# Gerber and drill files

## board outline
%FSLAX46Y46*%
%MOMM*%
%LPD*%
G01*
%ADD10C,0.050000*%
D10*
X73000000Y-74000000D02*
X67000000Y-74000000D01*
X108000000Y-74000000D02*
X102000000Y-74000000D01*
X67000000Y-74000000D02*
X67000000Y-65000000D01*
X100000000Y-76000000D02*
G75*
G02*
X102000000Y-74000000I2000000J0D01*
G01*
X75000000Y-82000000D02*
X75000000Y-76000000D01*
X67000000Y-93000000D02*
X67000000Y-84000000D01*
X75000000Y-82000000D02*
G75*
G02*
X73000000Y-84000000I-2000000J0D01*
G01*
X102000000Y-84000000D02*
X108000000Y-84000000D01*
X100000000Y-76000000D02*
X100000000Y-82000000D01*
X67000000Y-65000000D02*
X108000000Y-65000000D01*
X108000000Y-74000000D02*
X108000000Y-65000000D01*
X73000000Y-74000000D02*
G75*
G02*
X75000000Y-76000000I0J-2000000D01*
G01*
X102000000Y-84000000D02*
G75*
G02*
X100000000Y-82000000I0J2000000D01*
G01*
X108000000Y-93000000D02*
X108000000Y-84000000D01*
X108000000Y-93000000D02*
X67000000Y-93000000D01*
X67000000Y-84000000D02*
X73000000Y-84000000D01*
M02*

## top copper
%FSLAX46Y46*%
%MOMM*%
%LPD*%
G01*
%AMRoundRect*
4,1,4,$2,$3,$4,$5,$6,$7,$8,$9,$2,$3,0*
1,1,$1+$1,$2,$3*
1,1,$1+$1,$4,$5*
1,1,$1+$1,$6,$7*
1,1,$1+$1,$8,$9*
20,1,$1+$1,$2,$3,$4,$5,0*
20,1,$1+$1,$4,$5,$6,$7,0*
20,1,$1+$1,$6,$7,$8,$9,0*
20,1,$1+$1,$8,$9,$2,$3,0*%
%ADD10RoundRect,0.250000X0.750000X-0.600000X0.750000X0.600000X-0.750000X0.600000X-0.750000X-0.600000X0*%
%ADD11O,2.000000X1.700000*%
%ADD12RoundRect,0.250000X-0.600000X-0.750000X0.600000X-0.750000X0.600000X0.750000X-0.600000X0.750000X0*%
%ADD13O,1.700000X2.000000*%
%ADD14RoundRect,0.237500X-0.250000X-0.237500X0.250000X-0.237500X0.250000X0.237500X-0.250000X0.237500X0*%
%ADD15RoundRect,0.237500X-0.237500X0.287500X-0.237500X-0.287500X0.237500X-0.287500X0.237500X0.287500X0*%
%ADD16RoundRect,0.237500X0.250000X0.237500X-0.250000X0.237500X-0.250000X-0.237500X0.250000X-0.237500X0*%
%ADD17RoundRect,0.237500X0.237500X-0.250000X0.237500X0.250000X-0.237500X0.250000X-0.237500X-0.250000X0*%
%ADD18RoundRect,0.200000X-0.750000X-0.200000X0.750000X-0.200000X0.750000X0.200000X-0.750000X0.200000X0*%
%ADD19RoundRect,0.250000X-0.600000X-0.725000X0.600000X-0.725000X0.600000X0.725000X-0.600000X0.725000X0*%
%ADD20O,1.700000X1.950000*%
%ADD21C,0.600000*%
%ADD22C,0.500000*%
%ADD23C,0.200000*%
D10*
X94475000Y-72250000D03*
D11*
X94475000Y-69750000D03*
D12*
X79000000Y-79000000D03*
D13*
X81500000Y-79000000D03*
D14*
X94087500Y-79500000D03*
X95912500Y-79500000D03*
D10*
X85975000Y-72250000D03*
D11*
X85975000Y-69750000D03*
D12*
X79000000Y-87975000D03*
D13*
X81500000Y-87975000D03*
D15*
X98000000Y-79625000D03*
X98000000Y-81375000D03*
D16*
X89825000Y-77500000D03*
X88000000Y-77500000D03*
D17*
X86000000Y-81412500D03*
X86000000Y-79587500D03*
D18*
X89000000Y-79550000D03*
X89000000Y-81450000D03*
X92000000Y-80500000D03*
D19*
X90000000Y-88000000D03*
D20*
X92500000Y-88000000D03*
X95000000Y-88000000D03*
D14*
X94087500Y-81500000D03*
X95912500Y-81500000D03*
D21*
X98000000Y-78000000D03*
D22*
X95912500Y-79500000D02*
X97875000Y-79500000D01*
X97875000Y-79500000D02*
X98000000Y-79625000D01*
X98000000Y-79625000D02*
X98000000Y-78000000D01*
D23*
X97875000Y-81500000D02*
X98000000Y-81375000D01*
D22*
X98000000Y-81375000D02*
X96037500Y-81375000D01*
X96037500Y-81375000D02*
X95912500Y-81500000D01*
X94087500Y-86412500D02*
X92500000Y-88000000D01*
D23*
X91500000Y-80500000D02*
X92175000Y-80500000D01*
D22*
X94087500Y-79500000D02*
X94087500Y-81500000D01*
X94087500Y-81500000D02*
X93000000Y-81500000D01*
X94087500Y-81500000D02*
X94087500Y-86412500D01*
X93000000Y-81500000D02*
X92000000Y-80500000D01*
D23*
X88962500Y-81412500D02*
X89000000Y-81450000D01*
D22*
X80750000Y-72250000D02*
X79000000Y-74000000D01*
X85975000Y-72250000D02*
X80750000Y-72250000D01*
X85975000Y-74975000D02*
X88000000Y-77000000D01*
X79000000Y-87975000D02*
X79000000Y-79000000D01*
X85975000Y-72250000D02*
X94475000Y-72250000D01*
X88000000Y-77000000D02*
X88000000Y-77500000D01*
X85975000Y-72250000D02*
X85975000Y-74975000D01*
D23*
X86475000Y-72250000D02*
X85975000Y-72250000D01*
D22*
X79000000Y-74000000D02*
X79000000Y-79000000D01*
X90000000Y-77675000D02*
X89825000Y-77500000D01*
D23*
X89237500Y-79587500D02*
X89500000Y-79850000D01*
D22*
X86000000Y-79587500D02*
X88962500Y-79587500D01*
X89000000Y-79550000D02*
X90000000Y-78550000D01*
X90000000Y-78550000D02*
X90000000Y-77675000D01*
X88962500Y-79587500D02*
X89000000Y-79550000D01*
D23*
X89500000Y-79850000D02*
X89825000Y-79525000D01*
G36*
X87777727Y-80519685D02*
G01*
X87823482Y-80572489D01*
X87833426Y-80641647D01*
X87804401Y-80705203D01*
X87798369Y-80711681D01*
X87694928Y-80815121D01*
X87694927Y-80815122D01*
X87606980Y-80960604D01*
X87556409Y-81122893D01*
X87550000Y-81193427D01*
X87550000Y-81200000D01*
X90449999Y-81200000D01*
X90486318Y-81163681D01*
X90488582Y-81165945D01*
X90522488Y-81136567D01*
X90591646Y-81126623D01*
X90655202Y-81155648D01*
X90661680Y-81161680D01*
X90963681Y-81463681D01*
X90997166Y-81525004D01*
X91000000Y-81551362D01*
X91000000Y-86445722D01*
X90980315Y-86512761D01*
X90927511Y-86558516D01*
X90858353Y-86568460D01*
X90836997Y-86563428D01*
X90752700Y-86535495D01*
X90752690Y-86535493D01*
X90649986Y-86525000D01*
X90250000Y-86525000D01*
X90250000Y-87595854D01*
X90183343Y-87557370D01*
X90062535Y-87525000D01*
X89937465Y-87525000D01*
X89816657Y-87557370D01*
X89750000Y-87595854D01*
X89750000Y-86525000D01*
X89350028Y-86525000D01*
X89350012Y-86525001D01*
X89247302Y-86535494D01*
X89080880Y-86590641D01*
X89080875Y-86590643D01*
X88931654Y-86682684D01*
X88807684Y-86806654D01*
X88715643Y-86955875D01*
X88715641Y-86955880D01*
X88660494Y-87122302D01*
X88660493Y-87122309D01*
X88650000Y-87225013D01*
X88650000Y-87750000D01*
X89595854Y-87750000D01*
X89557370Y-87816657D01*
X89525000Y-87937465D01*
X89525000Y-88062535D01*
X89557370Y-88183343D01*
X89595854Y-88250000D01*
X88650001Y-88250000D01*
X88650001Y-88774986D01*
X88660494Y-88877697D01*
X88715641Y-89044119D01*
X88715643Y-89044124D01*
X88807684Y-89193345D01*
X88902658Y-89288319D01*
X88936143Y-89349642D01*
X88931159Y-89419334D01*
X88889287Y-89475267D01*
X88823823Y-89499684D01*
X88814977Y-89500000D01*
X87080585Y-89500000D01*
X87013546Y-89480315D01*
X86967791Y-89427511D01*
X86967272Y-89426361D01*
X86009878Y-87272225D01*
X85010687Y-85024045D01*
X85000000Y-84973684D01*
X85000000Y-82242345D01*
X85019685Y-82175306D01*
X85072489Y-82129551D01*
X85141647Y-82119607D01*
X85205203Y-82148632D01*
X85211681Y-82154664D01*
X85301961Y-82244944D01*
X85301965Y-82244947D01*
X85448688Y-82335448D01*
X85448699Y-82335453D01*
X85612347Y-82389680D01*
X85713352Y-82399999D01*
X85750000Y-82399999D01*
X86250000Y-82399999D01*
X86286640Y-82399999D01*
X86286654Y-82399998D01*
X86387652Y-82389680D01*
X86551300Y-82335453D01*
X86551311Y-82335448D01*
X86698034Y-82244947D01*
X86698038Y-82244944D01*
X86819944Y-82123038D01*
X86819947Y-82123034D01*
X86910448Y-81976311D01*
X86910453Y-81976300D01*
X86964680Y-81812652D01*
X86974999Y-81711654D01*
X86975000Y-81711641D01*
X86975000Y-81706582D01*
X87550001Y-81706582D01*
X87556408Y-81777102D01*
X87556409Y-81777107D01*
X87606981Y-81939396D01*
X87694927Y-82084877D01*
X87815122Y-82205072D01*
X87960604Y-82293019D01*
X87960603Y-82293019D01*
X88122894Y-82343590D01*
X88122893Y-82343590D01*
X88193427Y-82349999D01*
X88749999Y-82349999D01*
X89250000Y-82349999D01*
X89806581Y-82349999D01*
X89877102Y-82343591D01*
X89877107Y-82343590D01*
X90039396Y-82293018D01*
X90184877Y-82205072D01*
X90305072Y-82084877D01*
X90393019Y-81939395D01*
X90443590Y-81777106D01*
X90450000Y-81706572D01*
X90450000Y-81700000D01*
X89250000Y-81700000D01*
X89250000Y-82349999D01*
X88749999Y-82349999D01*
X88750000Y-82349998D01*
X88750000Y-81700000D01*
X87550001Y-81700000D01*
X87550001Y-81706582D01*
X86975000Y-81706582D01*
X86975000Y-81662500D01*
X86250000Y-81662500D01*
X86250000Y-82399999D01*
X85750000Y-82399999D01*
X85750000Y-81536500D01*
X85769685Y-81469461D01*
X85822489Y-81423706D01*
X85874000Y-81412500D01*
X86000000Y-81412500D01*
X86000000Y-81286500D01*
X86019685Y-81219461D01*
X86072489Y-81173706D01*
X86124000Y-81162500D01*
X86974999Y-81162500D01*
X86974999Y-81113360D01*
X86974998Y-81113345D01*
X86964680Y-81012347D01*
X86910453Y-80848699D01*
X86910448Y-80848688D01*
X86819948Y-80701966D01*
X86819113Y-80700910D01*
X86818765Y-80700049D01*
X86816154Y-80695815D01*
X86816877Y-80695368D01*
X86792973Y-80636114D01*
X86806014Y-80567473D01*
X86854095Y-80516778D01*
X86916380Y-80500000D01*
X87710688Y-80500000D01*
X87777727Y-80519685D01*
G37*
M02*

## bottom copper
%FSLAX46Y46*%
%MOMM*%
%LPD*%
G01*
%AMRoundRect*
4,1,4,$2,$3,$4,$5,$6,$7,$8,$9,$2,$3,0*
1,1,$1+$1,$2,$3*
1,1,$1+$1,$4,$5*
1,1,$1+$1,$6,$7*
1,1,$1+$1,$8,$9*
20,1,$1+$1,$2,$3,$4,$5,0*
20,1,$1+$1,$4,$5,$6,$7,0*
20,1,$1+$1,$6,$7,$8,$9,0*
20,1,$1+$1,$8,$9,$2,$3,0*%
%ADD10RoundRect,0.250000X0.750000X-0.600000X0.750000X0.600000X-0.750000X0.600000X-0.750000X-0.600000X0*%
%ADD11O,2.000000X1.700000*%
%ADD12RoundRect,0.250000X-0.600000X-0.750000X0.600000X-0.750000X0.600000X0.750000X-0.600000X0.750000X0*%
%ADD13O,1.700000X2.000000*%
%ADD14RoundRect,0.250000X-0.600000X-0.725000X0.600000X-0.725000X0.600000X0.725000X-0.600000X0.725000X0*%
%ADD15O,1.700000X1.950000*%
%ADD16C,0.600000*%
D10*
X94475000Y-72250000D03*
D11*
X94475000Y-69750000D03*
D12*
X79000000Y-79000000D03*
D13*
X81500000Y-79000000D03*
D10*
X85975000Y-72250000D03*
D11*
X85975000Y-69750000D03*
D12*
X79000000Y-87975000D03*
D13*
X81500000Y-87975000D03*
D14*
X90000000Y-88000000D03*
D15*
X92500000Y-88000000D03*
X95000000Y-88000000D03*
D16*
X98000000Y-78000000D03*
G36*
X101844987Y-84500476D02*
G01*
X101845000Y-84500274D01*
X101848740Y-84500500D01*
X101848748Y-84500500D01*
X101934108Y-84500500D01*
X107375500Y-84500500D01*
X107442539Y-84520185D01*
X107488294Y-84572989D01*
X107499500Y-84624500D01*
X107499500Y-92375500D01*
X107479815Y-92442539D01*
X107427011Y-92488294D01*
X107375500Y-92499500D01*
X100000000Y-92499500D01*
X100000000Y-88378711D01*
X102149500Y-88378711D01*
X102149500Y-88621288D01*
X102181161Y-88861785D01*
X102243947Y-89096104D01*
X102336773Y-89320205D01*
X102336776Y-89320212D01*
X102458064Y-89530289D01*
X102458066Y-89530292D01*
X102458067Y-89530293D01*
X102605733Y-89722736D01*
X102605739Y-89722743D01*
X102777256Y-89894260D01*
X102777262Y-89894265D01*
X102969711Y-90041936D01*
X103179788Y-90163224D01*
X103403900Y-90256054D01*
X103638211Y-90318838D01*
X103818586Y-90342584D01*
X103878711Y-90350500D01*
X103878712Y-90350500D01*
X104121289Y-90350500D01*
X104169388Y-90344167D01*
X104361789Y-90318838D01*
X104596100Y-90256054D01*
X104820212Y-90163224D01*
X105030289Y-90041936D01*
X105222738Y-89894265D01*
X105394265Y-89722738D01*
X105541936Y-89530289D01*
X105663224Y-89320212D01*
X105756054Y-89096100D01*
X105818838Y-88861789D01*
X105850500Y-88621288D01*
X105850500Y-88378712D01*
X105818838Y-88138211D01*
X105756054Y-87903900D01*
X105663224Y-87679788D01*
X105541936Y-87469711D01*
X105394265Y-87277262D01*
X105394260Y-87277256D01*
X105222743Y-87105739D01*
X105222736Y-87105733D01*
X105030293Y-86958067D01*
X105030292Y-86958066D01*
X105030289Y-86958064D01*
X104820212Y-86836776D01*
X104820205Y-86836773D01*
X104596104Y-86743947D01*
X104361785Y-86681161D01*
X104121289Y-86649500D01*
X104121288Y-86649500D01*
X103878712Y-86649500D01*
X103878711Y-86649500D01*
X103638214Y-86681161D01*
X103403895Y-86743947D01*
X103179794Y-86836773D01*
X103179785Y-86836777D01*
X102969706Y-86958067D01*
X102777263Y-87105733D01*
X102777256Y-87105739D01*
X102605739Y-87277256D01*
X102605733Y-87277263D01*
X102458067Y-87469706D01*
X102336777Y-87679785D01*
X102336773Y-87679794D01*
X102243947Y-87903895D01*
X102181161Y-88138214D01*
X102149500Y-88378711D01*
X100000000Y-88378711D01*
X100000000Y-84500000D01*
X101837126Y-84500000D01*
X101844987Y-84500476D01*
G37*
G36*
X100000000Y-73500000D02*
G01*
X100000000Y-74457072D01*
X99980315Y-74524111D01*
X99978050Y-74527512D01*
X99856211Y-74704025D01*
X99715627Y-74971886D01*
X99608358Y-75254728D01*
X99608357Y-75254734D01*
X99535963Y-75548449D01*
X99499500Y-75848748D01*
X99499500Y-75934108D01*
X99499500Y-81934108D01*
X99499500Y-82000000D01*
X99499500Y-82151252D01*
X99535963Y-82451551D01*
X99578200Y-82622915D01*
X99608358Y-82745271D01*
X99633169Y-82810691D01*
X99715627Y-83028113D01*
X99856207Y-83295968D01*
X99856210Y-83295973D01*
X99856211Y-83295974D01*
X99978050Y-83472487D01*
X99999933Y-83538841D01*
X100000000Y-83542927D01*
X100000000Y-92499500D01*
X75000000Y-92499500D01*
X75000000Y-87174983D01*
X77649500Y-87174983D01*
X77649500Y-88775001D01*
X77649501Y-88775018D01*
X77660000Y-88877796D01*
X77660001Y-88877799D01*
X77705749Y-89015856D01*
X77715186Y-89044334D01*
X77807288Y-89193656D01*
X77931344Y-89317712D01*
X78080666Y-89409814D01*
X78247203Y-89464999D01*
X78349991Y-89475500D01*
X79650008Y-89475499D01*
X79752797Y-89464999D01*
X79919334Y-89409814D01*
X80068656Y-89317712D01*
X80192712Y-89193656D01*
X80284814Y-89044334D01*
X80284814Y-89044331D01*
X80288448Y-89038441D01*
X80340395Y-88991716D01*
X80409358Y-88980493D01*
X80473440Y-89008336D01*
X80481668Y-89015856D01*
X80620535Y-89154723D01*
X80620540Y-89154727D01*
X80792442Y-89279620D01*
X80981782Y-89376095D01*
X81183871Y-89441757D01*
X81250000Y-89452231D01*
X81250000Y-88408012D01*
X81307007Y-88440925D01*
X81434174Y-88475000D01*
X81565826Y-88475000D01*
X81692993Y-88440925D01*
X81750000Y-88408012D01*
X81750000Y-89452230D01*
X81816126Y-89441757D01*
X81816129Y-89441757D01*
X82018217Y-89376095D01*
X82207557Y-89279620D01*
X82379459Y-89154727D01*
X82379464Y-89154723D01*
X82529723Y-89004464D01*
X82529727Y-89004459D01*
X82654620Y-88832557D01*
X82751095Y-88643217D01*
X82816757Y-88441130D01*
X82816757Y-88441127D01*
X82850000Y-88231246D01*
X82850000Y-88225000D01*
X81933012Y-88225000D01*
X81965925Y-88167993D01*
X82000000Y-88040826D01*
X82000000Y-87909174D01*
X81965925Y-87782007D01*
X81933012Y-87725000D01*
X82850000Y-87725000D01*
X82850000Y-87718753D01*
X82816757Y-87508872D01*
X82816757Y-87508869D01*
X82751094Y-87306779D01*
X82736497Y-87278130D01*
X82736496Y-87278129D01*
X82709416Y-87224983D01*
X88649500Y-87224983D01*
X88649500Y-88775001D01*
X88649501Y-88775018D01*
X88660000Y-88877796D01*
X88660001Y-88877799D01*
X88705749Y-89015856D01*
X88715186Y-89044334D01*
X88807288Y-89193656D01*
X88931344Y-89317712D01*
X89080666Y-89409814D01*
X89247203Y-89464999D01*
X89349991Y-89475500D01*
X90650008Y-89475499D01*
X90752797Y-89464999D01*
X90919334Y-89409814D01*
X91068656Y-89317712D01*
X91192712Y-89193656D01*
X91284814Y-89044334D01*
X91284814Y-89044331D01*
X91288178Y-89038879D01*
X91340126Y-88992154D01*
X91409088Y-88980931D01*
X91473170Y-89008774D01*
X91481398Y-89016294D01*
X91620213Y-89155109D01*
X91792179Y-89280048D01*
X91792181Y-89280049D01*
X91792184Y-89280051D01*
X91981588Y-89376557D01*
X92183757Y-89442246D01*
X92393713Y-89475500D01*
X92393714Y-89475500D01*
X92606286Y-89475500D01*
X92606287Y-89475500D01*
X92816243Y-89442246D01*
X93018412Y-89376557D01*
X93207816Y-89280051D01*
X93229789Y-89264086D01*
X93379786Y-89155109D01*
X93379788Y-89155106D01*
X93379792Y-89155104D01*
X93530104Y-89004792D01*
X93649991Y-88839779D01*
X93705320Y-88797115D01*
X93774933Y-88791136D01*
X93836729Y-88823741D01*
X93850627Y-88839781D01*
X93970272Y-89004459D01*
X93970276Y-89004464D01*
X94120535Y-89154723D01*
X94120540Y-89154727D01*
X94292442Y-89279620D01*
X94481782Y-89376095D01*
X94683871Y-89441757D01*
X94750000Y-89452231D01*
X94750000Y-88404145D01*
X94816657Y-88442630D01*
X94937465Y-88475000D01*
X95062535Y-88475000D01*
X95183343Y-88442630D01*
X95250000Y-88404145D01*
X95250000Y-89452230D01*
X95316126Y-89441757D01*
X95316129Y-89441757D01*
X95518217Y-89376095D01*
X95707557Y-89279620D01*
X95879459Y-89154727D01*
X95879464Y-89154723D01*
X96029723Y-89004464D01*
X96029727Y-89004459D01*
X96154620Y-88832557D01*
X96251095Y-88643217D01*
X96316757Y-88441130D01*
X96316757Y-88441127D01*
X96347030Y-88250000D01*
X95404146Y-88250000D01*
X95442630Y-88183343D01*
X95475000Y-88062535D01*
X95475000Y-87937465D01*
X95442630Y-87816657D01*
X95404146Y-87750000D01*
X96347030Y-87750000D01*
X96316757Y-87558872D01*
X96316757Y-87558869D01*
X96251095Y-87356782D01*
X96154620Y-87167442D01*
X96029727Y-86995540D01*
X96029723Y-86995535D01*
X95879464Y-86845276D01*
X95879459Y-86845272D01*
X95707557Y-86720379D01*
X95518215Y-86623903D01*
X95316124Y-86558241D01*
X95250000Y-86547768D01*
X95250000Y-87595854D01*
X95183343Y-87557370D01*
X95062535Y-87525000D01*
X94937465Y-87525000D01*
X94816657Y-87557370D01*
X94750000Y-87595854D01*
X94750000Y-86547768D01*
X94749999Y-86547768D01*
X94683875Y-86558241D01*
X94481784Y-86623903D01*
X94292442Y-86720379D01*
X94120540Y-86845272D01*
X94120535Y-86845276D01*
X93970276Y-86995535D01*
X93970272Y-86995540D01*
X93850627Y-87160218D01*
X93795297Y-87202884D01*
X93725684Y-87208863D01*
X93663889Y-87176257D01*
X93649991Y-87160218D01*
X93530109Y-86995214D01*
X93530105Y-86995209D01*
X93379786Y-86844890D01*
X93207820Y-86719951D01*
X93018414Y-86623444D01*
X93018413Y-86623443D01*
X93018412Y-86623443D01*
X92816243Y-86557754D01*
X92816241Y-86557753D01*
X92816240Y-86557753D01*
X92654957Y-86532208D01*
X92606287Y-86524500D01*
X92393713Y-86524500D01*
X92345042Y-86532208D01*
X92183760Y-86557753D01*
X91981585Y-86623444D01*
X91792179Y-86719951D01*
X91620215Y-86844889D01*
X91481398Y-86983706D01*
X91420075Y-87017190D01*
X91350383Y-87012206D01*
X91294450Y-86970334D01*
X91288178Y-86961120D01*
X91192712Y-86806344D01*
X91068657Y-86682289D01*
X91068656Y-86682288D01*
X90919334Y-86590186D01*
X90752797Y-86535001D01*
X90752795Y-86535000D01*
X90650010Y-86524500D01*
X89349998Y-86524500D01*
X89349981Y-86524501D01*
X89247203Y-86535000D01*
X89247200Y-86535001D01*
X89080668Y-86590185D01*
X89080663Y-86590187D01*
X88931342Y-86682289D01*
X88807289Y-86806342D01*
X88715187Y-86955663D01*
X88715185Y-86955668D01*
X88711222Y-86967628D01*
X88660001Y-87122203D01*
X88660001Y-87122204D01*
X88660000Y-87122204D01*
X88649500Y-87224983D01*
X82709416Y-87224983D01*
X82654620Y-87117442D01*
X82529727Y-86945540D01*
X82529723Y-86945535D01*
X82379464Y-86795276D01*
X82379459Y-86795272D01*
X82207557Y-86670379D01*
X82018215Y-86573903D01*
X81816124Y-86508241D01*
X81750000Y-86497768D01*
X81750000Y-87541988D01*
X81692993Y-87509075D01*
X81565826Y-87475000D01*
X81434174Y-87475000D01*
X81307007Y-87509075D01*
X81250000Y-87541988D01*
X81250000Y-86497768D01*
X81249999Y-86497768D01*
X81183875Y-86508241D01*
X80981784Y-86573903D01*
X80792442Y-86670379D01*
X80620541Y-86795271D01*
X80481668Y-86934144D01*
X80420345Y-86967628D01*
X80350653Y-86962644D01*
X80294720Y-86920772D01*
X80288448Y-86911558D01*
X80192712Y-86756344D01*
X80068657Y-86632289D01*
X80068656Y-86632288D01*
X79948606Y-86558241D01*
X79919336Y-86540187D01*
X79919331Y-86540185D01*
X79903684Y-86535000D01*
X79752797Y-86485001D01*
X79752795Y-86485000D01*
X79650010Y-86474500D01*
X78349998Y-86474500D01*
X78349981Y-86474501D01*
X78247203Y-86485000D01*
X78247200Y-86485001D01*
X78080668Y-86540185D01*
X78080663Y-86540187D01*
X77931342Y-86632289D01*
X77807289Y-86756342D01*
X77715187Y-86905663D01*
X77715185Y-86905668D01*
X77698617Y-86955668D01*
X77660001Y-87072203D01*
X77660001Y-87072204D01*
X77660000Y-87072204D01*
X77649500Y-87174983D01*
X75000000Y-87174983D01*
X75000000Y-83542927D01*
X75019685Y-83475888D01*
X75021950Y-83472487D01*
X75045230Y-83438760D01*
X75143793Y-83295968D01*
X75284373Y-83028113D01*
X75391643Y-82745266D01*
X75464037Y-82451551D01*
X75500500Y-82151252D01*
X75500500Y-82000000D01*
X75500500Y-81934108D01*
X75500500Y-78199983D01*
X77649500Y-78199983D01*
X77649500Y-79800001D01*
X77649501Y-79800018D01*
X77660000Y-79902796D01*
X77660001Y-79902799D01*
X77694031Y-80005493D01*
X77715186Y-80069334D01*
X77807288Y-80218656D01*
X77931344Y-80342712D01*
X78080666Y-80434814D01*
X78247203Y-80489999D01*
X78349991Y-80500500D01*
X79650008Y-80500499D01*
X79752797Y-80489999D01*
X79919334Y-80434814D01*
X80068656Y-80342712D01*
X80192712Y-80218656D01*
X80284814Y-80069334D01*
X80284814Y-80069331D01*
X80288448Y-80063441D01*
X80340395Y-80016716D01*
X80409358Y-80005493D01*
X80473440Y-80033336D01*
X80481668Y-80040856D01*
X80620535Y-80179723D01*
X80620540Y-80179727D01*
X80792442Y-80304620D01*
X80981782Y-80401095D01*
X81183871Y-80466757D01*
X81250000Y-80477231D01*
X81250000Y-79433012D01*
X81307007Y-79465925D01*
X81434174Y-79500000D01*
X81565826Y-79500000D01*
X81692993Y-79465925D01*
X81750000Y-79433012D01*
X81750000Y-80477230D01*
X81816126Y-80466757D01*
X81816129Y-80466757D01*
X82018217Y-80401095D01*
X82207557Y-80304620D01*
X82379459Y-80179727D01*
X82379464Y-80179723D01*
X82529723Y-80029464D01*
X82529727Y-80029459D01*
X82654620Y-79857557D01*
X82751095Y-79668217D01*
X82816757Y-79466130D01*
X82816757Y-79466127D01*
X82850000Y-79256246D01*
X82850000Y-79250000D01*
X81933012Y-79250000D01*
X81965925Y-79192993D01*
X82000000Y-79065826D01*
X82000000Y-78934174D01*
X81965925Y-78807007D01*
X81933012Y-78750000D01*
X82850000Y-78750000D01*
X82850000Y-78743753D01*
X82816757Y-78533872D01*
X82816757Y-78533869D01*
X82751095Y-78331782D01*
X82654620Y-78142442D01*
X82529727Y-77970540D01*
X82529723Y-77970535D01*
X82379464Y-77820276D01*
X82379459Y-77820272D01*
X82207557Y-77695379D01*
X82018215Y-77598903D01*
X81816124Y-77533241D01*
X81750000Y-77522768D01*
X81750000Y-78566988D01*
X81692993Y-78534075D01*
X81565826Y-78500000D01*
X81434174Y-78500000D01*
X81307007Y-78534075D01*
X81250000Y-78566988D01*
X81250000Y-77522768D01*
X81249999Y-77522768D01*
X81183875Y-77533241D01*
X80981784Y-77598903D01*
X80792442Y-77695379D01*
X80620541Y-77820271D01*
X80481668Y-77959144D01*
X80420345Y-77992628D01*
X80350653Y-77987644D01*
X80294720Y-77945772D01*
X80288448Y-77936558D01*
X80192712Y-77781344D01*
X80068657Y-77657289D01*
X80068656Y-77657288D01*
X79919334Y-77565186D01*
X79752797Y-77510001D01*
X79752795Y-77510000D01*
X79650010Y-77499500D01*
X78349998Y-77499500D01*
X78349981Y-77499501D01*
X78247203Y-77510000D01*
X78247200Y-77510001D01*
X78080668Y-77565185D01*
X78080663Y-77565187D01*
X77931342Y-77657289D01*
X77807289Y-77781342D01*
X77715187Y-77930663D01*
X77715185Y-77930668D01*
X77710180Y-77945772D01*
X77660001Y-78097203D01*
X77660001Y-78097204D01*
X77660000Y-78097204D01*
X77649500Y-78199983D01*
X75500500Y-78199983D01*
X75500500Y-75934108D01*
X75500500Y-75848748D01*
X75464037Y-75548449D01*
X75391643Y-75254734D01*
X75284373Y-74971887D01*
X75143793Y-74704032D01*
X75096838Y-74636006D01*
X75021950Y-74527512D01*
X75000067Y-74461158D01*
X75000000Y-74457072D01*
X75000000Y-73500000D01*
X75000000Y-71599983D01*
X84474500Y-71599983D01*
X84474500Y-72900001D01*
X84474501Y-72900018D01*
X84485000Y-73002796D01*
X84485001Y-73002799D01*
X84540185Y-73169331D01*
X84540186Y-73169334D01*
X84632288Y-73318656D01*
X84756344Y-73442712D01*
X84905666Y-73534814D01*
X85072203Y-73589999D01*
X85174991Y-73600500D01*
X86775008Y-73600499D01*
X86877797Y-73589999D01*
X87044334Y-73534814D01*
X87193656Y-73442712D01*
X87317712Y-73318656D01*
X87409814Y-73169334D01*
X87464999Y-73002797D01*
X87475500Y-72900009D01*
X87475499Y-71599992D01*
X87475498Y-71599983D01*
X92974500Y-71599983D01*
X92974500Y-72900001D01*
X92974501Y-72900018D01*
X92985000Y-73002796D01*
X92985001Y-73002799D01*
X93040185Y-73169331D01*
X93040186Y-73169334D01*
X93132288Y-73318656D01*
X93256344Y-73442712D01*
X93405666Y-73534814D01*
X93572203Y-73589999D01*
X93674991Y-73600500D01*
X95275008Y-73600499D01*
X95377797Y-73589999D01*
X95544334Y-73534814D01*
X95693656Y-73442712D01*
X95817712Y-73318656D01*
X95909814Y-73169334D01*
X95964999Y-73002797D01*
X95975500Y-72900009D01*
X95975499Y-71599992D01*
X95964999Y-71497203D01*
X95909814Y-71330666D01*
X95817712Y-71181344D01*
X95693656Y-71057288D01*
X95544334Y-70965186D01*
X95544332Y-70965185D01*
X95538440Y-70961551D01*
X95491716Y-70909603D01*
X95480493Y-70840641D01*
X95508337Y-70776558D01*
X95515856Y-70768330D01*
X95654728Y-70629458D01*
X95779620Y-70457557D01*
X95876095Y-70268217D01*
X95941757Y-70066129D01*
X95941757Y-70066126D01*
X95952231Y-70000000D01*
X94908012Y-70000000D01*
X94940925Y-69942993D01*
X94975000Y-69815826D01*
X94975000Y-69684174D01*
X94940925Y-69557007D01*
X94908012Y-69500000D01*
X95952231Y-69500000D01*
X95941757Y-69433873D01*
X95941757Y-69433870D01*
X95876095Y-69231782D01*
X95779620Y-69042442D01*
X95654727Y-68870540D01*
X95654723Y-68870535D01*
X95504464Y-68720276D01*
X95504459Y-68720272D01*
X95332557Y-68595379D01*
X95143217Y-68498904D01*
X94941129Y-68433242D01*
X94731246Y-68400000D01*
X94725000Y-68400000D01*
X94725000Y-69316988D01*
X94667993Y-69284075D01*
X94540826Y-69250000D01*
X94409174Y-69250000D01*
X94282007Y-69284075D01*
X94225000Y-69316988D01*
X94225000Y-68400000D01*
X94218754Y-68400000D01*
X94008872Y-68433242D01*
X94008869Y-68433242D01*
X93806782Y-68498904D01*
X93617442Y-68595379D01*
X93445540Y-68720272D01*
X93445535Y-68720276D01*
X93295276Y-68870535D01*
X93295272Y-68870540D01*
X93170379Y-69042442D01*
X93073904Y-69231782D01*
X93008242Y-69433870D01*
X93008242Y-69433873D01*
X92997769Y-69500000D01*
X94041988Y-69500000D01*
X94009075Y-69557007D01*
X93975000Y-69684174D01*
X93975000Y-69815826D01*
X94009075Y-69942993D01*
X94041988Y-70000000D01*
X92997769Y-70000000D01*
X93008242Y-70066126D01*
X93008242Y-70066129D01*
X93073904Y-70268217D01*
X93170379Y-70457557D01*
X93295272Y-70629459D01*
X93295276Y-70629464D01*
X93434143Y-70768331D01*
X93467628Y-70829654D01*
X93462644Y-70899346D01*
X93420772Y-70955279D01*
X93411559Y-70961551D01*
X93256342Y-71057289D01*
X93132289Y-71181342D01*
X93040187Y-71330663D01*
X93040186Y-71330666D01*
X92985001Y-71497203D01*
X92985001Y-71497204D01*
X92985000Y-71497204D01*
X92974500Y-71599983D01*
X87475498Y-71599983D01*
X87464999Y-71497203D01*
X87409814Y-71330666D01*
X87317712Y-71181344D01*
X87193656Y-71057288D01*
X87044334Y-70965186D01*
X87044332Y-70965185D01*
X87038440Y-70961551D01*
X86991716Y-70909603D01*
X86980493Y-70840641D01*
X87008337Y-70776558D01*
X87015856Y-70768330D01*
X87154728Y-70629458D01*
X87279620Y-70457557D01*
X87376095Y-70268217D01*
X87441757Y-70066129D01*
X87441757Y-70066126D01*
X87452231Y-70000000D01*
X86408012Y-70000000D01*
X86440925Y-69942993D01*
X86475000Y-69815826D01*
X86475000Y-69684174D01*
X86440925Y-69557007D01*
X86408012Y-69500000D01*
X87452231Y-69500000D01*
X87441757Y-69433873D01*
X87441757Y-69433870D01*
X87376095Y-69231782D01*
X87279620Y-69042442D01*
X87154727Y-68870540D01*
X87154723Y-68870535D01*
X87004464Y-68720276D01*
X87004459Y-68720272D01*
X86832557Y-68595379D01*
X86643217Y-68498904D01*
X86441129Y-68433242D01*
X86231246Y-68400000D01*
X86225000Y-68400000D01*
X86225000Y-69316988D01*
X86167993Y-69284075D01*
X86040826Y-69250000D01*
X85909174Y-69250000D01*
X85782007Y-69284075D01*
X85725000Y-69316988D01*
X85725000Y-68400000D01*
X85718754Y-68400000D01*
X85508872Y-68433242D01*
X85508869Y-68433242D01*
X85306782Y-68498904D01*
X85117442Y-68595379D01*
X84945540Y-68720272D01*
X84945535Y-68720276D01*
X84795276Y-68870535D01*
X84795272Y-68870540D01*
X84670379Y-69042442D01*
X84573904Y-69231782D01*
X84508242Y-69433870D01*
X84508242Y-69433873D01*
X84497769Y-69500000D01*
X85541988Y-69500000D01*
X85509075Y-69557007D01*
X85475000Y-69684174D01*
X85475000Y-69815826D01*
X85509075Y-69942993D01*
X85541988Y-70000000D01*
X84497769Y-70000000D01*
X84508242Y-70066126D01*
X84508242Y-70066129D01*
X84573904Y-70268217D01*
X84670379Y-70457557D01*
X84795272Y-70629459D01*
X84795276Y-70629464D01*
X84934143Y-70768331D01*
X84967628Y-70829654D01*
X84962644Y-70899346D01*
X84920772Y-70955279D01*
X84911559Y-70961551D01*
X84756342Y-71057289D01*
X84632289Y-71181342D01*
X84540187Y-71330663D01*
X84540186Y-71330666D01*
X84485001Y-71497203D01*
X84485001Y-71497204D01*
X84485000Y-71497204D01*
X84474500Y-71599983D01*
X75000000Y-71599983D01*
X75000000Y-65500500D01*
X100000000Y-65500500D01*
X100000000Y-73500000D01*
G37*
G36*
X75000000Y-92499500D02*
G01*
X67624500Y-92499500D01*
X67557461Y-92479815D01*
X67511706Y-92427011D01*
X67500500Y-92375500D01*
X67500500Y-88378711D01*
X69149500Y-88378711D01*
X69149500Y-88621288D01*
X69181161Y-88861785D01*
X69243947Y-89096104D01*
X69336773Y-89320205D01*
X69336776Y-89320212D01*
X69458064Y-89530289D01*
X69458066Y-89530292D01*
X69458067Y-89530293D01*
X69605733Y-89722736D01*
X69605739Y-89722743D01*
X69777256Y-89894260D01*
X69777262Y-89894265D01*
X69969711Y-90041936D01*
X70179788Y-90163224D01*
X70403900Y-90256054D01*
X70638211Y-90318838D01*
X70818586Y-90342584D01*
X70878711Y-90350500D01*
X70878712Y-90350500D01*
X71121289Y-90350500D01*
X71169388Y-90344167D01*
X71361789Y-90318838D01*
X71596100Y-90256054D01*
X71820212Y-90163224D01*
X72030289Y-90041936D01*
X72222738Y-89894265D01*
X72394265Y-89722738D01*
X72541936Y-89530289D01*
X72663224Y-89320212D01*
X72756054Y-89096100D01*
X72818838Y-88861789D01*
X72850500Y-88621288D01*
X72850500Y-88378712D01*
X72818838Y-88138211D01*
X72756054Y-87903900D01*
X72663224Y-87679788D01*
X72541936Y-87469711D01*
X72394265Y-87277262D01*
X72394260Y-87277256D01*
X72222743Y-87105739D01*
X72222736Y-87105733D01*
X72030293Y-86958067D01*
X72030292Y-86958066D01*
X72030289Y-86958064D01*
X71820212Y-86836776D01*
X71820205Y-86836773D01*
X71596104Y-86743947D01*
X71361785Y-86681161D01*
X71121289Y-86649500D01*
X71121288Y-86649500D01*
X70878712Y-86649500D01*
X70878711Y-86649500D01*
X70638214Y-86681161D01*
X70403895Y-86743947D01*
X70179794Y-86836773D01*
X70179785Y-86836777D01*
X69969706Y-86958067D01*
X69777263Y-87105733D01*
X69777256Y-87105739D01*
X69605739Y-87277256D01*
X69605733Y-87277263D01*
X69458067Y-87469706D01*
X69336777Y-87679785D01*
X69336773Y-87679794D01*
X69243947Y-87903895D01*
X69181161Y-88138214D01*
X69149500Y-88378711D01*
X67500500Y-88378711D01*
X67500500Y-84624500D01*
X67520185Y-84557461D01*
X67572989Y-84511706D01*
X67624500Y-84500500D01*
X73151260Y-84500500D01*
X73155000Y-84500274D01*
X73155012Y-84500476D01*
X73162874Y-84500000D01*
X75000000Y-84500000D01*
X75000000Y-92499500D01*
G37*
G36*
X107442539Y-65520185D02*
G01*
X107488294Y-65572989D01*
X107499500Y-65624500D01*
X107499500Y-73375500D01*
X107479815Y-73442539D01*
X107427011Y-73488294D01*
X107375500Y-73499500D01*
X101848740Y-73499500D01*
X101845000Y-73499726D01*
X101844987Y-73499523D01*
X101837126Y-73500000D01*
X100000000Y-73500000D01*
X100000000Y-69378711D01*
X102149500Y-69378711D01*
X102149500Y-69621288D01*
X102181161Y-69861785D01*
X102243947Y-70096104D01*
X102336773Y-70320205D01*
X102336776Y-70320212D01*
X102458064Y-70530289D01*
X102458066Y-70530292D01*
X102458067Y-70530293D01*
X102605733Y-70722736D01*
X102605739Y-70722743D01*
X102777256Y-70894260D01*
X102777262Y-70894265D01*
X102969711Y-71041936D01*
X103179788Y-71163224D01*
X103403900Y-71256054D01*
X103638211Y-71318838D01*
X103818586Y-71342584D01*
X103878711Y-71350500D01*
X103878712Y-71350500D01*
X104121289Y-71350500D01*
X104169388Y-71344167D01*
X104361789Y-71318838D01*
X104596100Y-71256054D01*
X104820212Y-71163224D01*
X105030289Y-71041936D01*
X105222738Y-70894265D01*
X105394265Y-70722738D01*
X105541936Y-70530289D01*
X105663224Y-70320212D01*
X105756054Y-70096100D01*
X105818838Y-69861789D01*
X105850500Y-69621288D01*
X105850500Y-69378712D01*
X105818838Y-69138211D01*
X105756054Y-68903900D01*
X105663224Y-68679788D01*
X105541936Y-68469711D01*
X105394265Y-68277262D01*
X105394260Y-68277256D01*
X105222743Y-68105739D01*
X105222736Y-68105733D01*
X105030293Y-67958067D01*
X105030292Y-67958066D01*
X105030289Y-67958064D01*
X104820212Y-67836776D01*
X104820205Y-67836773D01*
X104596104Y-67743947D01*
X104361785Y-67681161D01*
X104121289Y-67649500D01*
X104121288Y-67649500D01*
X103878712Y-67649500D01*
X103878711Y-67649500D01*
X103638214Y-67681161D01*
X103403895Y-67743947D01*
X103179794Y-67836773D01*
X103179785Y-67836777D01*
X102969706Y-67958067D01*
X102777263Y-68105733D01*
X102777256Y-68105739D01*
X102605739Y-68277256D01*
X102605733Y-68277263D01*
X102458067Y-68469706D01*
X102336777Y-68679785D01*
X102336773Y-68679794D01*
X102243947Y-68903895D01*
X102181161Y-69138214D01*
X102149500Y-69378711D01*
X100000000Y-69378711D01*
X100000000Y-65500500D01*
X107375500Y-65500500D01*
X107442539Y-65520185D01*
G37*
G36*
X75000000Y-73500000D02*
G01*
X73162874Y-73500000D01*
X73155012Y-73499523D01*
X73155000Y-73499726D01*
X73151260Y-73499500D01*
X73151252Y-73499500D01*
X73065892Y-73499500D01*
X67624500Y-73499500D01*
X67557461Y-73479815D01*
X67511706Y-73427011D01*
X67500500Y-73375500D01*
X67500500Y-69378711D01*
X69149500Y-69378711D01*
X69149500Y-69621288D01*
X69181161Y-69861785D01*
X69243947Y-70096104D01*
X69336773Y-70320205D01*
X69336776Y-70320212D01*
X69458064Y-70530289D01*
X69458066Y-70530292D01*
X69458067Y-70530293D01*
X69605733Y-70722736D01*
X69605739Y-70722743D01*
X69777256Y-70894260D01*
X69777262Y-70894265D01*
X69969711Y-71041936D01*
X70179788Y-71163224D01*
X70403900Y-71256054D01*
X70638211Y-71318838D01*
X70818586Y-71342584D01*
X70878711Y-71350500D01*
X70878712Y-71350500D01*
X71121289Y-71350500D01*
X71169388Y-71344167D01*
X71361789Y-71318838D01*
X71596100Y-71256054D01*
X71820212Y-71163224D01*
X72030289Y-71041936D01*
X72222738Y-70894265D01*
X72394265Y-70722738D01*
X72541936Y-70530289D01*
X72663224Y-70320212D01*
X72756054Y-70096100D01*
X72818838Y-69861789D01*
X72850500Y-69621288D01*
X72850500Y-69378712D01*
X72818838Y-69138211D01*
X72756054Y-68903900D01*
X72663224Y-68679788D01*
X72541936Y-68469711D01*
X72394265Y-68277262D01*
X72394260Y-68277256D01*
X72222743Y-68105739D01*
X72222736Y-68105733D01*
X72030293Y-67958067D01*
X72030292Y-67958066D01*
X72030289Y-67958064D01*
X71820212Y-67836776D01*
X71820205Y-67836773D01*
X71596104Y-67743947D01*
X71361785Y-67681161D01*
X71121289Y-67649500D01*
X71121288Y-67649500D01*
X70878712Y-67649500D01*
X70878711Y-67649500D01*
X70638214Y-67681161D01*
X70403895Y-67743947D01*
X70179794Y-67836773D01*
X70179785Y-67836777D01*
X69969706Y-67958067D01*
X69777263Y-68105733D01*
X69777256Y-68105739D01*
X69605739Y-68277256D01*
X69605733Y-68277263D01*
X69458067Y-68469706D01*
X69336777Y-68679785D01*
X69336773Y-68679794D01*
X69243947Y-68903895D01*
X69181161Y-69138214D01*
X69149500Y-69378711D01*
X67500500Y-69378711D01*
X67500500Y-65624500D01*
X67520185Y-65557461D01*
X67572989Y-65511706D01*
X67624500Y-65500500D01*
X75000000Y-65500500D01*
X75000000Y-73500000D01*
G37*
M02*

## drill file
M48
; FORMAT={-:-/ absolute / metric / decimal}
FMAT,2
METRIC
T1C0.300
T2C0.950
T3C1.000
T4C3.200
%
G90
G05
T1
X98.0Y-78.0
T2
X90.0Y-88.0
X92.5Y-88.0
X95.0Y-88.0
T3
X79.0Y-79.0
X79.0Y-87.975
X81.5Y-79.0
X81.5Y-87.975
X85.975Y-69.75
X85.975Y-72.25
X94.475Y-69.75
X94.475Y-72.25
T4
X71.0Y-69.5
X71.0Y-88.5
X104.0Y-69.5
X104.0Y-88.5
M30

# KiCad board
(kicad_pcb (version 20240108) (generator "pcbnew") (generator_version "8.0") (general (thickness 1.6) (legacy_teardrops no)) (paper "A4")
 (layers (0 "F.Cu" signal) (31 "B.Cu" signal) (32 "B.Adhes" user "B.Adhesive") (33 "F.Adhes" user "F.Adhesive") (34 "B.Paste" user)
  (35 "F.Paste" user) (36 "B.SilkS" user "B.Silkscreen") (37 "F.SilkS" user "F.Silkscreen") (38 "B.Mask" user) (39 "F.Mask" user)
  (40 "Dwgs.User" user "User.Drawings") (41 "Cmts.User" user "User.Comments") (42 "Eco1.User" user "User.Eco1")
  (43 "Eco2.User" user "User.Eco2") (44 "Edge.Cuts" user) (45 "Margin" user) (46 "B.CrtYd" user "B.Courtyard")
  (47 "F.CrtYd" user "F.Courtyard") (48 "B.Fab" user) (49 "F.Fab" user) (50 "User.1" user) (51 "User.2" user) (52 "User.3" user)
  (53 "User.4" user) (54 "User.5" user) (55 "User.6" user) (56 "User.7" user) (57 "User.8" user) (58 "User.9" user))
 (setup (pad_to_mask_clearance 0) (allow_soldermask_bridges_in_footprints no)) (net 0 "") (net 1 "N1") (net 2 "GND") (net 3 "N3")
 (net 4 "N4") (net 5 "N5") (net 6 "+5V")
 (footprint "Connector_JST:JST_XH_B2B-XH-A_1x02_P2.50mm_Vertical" (layer "F.Cu") (at 94.475 72.25 90)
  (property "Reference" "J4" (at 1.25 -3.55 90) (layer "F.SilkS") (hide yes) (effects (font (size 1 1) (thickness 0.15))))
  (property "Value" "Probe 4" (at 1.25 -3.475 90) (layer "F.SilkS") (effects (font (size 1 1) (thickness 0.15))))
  (pad "1" thru_hole roundrect (at 0 0 90) (size 1.7 2) (drill 1) (layers "*.Cu" "*.Mask") (remove_unused_layers no)
   (roundrect_rratio 0.147059) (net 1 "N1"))
  (pad "2" thru_hole oval (at 2.5 0 90) (size 1.7 2) (drill 1) (layers "*.Cu" "*.Mask") (remove_unused_layers no) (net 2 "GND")))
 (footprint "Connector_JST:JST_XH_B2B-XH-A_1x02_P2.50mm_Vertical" (layer "F.Cu") (at 79 79)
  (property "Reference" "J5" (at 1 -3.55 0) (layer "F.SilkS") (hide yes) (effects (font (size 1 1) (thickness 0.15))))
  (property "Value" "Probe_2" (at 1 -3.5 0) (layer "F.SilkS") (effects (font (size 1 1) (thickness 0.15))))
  (pad "1" thru_hole roundrect (at 0 0) (size 1.7 2) (drill 1) (layers "*.Cu" "*.Mask") (remove_unused_layers no)
   (roundrect_rratio 0.147059) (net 1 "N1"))
  (pad "2" thru_hole oval (at 2.5 0) (size 1.7 2) (drill 1) (layers "*.Cu" "*.Mask") (remove_unused_layers no) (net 2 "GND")))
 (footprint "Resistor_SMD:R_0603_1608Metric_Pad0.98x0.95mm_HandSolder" (layer "F.Cu") (at 95 79.5)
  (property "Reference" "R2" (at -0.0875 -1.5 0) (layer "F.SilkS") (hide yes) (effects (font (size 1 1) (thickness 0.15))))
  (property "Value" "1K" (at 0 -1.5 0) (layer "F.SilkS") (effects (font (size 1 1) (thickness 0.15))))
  (pad "1" smd roundrect (at -0.9125 0) (size 0.975 0.95) (layers "F.Cu" "F.Paste" "F.Mask") (roundrect_rratio 0.25) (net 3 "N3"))
  (pad "2" smd roundrect (at 0.9125 0) (size 0.975 0.95) (layers "F.Cu" "F.Paste" "F.Mask") (roundrect_rratio 0.25) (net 2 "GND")))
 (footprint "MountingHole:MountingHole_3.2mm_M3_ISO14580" (layer "F.Cu") (at 71 88.5)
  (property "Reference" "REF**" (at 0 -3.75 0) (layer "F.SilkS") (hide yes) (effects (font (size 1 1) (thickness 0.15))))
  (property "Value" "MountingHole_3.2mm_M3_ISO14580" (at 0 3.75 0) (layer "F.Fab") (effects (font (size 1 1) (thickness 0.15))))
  (pad "" np_thru_hole circle (at 0 0) (size 3.2 3.2) (drill 3.2) (layers "*.Cu" "*.Mask")))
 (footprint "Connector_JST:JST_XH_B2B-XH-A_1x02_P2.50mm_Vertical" (layer "F.Cu") (at 85.975 72.25 90)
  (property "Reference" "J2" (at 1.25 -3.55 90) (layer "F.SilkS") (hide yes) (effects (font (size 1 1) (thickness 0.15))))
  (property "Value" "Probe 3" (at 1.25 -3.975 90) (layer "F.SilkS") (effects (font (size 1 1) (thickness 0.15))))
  (pad "1" thru_hole roundrect (at 0 0 90) (size 1.7 2) (drill 1) (layers "*.Cu" "*.Mask") (remove_unused_layers no)
   (roundrect_rratio 0.147059) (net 1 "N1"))
  (pad "2" thru_hole oval (at 2.5 0 90) (size 1.7 2) (drill 1) (layers "*.Cu" "*.Mask") (remove_unused_layers no) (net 2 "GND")))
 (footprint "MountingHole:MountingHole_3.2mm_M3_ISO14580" (layer "F.Cu") (at 71 69.5)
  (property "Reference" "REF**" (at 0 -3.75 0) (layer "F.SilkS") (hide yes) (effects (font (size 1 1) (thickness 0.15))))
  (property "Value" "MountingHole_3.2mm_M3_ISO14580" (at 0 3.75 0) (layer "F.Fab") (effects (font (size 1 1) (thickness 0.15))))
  (pad "" np_thru_hole circle (at 0 0) (size 3.2 3.2) (drill 3.2) (layers "*.Cu" "*.Mask")))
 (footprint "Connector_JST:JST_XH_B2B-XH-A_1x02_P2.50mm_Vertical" (layer "F.Cu") (at 79 87.975)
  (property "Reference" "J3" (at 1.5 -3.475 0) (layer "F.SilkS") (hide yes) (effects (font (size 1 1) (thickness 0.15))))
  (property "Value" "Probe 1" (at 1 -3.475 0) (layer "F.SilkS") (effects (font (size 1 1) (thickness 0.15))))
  (pad "1" thru_hole roundrect (at 0 0) (size 1.7 2) (drill 1) (layers "*.Cu" "*.Mask") (remove_unused_layers no)
   (roundrect_rratio 0.147059) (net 1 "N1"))
  (pad "2" thru_hole oval (at 2.5 0) (size 1.7 2) (drill 1) (layers "*.Cu" "*.Mask") (remove_unused_layers no) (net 2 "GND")))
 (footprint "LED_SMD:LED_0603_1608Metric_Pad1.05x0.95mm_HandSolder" (layer "F.Cu") (at 98 80.5 -90)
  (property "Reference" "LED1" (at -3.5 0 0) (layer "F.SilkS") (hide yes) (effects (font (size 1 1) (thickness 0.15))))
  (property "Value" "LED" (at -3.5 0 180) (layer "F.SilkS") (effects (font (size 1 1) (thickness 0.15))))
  (pad "1" smd roundrect (at -0.875 0 270) (size 1.05 0.95) (layers "F.Cu" "F.Paste" "F.Mask") (roundrect_rratio 0.25) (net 2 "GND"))
  (pad "2" smd roundrect (at 0.875 0 270) (size 1.05 0.95) (layers "F.Cu" "F.Paste" "F.Mask") (roundrect_rratio 0.25) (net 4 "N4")))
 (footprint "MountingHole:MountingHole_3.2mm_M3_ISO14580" (layer "F.Cu") (at 104 88.5)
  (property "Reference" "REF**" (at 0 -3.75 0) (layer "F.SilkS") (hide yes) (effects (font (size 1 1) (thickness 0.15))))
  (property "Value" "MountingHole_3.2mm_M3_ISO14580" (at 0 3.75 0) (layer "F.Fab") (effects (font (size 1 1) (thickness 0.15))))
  (pad "" np_thru_hole circle (at 0 0) (size 3.2 3.2) (drill 3.2) (layers "*.Cu" "*.Mask")))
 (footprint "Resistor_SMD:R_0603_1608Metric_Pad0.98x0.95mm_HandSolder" (layer "F.Cu") (at 88.9125 77.5 180)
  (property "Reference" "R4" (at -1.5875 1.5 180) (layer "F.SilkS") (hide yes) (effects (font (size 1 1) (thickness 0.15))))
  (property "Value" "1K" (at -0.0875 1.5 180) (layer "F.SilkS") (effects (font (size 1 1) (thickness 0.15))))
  (pad "1" smd roundrect (at -0.9125 0 180) (size 0.975 0.95) (layers "F.Cu" "F.Paste" "F.Mask") (roundrect_rratio 0.25) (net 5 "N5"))
  (pad "2" smd roundrect (at 0.9125 0 180) (size 0.975 0.95) (layers "F.Cu" "F.Paste" "F.Mask") (roundrect_rratio 0.25) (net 1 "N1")))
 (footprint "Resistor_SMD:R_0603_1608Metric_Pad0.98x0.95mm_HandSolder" (layer "F.Cu") (at 86 80.5 90)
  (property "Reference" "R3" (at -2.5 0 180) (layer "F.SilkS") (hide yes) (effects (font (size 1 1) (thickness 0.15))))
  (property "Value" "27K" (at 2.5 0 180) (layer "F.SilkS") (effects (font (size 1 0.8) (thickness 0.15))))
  (pad "1" smd roundrect (at -0.9125 0 90) (size 0.975 0.95) (layers "F.Cu" "F.Paste" "F.Mask") (roundrect_rratio 0.25) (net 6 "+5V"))
  (pad "2" smd roundrect (at 0.9125 0 90) (size 0.975 0.95) (layers "F.Cu" "F.Paste" "F.Mask") (roundrect_rratio 0.25) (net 5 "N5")))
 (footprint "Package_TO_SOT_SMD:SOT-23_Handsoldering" (layer "F.Cu") (at 90.5 80.5)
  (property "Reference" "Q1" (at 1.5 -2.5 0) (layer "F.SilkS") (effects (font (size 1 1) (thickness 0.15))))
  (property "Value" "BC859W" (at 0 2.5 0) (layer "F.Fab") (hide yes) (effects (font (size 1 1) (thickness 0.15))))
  (pad "1" smd roundrect (at -1.5 -0.95) (size 1.9 0.8) (layers "F.Cu" "F.Paste" "F.Mask") (roundrect_rratio 0.25) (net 5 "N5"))
  (pad "2" smd roundrect (at -1.5 0.95) (size 1.9 0.8) (layers "F.Cu" "F.Paste" "F.Mask") (roundrect_rratio 0.25) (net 6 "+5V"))
  (pad "3" smd roundrect (at 1.5 0) (size 1.9 0.8) (layers "F.Cu" "F.Paste" "F.Mask") (roundrect_rratio 0.25) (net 3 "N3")))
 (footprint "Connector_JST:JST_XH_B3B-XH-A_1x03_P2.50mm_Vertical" (layer "F.Cu") (at 90 88)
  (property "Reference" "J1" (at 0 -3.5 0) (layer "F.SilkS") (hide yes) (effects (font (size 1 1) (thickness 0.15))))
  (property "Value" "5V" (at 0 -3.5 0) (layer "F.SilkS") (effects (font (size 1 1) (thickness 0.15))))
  (pad "1" thru_hole roundrect (at 0 0) (size 1.7 1.95) (drill 0.95) (layers "*.Cu" "*.Mask") (remove_unused_layers no)
   (roundrect_rratio 0.147059) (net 6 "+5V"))
  (pad "2" thru_hole oval (at 2.5 0) (size 1.7 1.95) (drill 0.95) (layers "*.Cu" "*.Mask") (remove_unused_layers no) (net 3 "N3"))
  (pad "3" thru_hole oval (at 5 0) (size 1.7 1.95) (drill 0.95) (layers "*.Cu" "*.Mask") (remove_unused_layers no) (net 2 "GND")))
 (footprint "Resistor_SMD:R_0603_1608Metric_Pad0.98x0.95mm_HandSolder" (layer "F.Cu") (at 95 81.5)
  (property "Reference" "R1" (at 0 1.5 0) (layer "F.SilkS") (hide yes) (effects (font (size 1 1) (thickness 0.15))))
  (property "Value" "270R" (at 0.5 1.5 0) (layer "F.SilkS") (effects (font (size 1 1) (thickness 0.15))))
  (pad "1" smd roundrect (at -0.9125 0) (size 0.975 0.95) (layers "F.Cu" "F.Paste" "F.Mask") (roundrect_rratio 0.25) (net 3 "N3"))
  (pad "2" smd roundrect (at 0.9125 0) (size 0.975 0.95) (layers "F.Cu" "F.Paste" "F.Mask") (roundrect_rratio 0.25) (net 4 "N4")))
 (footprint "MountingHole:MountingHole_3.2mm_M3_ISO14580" (layer "F.Cu") (at 104 69.5)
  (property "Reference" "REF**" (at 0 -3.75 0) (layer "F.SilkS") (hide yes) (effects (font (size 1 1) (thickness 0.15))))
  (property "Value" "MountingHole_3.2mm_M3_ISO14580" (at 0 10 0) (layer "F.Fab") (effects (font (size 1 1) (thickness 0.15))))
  (pad "" np_thru_hole circle (at 0 0) (size 3.2 3.2) (drill 3.2) (layers "*.Cu" "*.Mask")))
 (gr_line (start 73 74) (end 67 74) (stroke (width 0.05) (type default)) (layer "Edge.Cuts"))
 (gr_line (start 108 74) (end 102 74) (stroke (width 0.05) (type default)) (layer "Edge.Cuts"))
 (gr_line (start 67 74) (end 67 65) (stroke (width 0.05) (type default)) (layer "Edge.Cuts"))
 (gr_arc (start 100 76) (mid 100.585786 74.585786) (end 102 74) (stroke (width 0.05) (type default)) (layer "Edge.Cuts"))
 (gr_line (start 75 82) (end 75 76) (stroke (width 0.05) (type default)) (layer "Edge.Cuts"))
 (gr_line (start 67 93) (end 67 84) (stroke (width 0.05) (type default)) (layer "Edge.Cuts"))
 (gr_arc (start 75 82) (mid 74.414214 83.414214) (end 73 84) (stroke (width 0.05) (type default)) (layer "Edge.Cuts"))
 (gr_line (start 102 84) (end 108 84) (stroke (width 0.05) (type default)) (layer "Edge.Cuts"))
 (gr_line (start 100 76) (end 100 82) (stroke (width 0.05) (type default)) (layer "Edge.Cuts"))
 (gr_line (start 67 65) (end 108 65) (stroke (width 0.05) (type default)) (layer "Edge.Cuts"))
 (gr_line (start 108 74) (end 108 65) (stroke (width 0.05) (type default)) (layer "Edge.Cuts"))
 (gr_arc (start 73 74) (mid 74.414214 74.585786) (end 75 76) (stroke (width 0.05) (type default)) (layer "Edge.Cuts"))
 (gr_arc (start 102 84) (mid 100.585786 83.414214) (end 100 82) (stroke (width 0.05) (type default)) (layer "Edge.Cuts"))
 (gr_line (start 108 93) (end 108 84) (stroke (width 0.05) (type default)) (layer "Edge.Cuts"))
 (gr_line (start 108 93) (end 67 93) (stroke (width 0.05) (type default)) (layer "Edge.Cuts"))
 (gr_line (start 67 84) (end 73 84) (stroke (width 0.05) (type default)) (layer "Edge.Cuts"))
 (segment (start 95.9125 79.5) (end 97.875 79.5) (width 0.5) (layer "F.Cu") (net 2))
 (segment (start 97.875 79.5) (end 98 79.625) (width 0.5) (layer "F.Cu") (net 2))
 (segment (start 98 79.625) (end 98 78) (width 0.5) (layer "F.Cu") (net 2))
 (via (at 98 78) (size 0.6) (drill 0.3) (layers "F.Cu" "B.Cu") (free yes) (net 2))
 (segment (start 97.875 81.5) (end 98 81.375) (width 0.2) (layer "F.Cu") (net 4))
 (segment (start 98 81.375) (end 96.0375 81.375) (width 0.5) (layer "F.Cu") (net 4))
 (segment (start 96.0375 81.375) (end 95.9125 81.5) (width 0.5) (layer "F.Cu") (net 4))
 (segment (start 94.0875 86.4125) (end 92.5 88) (width 0.5) (layer "F.Cu") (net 3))
 (segment (start 91.5 80.5) (end 92.175 80.5) (width 0.2) (layer "F.Cu") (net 3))
 (segment (start 94.0875 79.5) (end 94.0875 81.5) (width 0.5) (layer "F.Cu") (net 3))
 (segment (start 94.0875 81.5) (end 93 81.5) (width 0.5) (layer "F.Cu") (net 3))
 (segment (start 94.0875 81.5) (end 94.0875 86.4125) (width 0.5) (layer "F.Cu") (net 3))
 (segment (start 93 81.5) (end 92 80.5) (width 0.5) (layer "F.Cu") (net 3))
 (segment (start 88.9625 81.4125) (end 89 81.45) (width 0.2) (layer "F.Cu") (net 6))
 (segment (start 80.75 72.25) (end 79 74) (width 0.5) (layer "F.Cu") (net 1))
 (segment (start 85.975 72.25) (end 80.75 72.25) (width 0.5) (layer "F.Cu") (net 1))
 (segment (start 85.975 74.975) (end 88 77) (width 0.5) (layer "F.Cu") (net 1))
 (segment (start 79 87.975) (end 79 79) (width 0.5) (layer "F.Cu") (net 1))
 (segment (start 85.975 72.25) (end 94.475 72.25) (width 0.5) (layer "F.Cu") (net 1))
 (segment (start 88 77) (end 88 77.5) (width 0.5) (layer "F.Cu") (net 1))
 (segment (start 85.975 72.25) (end 85.975 74.975) (width 0.5) (layer "F.Cu") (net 1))
 (segment (start 86.475 72.25) (end 85.975 72.25) (width 0.2) (layer "F.Cu") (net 1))
 (segment (start 79 74) (end 79 79) (width 0.5) (layer "F.Cu") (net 1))
 (segment (start 90 77.675) (end 89.825 77.5) (width 0.5) (layer "F.Cu") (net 5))
 (segment (start 89.2375 79.5875) (end 89.5 79.85) (width 0.2) (layer "F.Cu") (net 5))
 (segment (start 86 79.5875) (end 88.9625 79.5875) (width 0.5) (layer "F.Cu") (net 5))
 (segment (start 89 79.55) (end 90 78.55) (width 0.5) (layer "F.Cu") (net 5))
 (segment (start 90 78.55) (end 90 77.675) (width 0.5) (layer "F.Cu") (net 5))
 (segment (start 88.9625 79.5875) (end 89 79.55) (width 0.5) (layer "F.Cu") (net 5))
 (segment (start 89.5 79.85) (end 89.825 79.525) (width 0.2) (layer "F.Cu") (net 5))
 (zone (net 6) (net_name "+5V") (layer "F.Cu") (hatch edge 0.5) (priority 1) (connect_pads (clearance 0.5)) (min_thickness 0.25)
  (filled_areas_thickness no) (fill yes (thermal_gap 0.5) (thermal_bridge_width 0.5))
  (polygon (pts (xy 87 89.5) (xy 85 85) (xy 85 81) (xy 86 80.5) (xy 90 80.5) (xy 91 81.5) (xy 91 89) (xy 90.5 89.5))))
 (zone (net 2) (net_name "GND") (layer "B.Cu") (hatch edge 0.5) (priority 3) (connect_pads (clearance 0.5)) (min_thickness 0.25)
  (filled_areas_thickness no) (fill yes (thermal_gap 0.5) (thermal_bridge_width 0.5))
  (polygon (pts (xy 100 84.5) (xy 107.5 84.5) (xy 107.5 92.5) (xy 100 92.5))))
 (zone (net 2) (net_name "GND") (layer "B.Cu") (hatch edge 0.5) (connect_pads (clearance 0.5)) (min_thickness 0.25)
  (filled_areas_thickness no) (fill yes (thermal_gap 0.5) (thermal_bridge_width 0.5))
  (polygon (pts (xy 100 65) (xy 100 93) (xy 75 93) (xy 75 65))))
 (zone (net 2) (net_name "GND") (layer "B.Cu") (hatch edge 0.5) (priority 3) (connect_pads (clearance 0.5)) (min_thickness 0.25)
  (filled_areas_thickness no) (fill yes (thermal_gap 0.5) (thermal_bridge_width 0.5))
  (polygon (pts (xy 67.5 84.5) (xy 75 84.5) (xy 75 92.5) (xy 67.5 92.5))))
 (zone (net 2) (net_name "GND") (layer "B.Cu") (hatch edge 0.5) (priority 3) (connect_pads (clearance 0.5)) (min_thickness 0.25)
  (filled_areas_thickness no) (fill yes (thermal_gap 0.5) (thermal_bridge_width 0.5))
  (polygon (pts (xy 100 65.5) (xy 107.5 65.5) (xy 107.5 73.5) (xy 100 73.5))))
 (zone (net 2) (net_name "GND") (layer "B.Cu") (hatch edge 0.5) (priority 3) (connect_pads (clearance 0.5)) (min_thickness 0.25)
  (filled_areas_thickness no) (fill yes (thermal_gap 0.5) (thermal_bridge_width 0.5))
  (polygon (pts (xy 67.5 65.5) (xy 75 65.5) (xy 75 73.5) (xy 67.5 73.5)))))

